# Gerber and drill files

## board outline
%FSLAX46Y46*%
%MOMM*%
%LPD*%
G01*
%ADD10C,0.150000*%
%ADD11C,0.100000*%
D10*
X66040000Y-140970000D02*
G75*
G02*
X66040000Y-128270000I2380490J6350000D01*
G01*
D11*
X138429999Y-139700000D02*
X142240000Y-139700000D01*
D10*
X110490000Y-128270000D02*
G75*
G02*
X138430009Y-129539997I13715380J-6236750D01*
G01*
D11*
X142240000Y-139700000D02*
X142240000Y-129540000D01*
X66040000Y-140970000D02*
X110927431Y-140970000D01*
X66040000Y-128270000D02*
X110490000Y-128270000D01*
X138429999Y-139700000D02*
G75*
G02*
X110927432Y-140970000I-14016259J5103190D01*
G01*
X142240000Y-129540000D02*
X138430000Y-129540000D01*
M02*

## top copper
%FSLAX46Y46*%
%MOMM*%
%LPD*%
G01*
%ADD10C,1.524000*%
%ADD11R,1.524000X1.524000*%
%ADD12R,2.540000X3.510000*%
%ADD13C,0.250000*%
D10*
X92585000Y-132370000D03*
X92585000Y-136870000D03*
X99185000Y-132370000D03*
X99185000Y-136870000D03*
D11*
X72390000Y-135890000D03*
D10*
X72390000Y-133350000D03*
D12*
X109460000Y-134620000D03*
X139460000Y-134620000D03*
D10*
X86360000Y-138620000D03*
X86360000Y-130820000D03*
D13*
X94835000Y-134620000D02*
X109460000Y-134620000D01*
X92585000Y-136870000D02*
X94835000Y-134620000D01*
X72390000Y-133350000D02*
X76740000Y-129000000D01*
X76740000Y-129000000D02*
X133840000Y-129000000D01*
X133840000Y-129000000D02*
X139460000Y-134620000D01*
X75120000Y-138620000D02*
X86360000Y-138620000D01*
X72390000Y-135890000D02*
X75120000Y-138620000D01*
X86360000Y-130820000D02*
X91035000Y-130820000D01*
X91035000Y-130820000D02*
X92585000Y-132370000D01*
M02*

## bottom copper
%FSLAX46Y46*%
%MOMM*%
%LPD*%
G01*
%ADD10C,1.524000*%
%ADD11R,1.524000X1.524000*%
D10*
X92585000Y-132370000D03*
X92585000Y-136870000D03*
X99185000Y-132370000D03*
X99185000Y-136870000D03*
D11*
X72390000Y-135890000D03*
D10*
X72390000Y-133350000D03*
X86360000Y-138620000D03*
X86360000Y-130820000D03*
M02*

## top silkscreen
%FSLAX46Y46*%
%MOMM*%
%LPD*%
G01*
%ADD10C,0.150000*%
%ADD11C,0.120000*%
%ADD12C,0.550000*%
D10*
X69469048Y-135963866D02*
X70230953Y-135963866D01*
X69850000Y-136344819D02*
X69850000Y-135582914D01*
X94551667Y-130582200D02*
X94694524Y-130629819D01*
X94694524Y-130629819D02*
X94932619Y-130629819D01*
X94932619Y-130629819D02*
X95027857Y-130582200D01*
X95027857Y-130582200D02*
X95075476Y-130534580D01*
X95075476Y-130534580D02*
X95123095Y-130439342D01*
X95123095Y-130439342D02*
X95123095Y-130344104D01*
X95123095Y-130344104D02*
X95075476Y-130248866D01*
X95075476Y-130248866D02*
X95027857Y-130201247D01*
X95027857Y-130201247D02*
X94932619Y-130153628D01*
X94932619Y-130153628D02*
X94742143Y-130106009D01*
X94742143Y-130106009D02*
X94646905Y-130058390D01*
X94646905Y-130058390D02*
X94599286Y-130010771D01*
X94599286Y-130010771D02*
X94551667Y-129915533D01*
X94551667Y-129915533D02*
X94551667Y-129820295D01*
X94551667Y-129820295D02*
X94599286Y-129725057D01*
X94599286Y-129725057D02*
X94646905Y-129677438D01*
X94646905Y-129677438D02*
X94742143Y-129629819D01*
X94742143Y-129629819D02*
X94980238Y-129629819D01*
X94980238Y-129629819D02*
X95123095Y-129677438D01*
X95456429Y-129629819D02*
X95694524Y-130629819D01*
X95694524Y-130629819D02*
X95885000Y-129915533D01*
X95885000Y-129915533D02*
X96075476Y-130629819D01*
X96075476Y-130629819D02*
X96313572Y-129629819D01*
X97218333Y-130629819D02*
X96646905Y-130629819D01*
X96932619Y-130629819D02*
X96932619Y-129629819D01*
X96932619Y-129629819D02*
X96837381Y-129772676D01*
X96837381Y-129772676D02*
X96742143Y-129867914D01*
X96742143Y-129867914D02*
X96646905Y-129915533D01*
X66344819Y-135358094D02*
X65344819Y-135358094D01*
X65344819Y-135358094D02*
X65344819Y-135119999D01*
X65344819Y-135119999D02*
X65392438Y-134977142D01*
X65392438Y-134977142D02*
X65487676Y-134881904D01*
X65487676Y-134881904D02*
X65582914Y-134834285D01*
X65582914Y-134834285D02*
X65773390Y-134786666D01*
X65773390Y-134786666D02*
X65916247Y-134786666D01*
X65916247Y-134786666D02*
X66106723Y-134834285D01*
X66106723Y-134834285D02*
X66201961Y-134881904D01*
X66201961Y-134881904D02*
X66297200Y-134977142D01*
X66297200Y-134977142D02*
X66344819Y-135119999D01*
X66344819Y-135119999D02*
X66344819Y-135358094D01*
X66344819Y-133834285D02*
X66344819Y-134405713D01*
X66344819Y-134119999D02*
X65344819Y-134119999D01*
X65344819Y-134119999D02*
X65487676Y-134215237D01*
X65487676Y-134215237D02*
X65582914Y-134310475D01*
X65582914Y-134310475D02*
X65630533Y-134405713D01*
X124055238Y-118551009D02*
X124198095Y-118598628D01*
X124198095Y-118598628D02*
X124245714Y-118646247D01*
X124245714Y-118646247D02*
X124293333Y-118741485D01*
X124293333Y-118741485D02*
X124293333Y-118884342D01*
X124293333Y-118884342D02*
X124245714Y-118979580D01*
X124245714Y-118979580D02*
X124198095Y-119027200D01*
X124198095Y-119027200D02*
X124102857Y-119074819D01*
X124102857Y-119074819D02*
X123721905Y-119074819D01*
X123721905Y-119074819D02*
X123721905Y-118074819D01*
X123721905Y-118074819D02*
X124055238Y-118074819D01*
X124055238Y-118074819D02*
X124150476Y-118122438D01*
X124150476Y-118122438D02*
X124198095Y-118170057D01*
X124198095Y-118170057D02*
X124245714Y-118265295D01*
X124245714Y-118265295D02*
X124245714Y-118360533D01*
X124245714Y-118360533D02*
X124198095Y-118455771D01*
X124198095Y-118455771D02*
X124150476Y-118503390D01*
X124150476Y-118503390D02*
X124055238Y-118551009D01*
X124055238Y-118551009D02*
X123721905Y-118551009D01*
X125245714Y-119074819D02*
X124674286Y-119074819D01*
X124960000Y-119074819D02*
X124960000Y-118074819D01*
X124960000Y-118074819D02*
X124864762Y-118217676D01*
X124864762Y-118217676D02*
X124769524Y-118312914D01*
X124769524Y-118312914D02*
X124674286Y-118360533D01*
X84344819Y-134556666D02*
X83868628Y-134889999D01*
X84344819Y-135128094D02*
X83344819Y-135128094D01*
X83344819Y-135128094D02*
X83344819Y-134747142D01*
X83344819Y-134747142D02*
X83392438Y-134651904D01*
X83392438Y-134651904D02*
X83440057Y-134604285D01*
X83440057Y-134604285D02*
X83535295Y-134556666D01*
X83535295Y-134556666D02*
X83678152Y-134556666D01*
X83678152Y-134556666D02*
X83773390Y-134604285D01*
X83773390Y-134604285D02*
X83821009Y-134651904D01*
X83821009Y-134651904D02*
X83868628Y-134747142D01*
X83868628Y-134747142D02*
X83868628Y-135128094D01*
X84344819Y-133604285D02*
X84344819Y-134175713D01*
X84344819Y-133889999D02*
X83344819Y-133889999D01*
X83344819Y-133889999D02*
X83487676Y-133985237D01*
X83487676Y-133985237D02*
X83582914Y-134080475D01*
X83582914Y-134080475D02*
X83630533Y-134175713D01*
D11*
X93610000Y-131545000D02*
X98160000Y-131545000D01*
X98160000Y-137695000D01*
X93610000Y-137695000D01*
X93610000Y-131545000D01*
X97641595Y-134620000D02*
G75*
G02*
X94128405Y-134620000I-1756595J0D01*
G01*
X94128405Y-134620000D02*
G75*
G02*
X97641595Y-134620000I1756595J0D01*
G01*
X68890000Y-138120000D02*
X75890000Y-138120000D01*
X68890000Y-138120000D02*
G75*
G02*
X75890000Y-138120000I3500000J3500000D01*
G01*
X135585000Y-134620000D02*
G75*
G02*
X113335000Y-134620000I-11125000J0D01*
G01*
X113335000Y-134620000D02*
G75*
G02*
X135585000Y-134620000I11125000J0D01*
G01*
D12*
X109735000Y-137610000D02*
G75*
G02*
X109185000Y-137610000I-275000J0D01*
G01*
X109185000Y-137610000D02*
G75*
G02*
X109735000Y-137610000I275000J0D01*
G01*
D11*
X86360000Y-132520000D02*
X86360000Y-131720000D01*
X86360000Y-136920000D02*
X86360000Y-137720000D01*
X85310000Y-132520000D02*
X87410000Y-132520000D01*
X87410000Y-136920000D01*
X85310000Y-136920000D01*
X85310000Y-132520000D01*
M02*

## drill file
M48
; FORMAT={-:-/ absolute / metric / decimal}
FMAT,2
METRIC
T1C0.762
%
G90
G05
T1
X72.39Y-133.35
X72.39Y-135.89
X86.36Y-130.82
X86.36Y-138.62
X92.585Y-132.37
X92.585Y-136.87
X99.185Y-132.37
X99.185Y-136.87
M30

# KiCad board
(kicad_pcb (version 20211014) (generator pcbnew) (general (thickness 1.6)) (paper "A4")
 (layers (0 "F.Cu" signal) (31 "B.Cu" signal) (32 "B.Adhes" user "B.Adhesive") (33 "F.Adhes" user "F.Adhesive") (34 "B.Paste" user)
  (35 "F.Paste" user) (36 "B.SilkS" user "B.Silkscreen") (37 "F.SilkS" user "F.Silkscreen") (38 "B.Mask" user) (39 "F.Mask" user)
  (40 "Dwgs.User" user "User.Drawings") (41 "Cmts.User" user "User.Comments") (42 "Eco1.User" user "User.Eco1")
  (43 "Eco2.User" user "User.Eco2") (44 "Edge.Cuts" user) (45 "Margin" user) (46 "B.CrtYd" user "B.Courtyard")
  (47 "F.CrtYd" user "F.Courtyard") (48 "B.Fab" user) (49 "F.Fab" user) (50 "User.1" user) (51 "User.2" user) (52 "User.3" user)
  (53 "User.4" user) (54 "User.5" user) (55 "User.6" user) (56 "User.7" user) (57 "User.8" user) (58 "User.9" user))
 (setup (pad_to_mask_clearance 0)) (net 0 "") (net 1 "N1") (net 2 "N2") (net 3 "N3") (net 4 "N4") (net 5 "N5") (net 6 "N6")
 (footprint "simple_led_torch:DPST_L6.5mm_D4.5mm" (layer "F.Cu") (at 95.885 134.62)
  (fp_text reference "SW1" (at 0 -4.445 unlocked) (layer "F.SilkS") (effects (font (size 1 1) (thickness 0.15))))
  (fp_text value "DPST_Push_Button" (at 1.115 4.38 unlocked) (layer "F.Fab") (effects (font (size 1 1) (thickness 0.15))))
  (fp_rect (start -2.275 -3.075) (end 2.275 3.075) (layer "F.SilkS") (width 0.12) (fill none))
  (fp_circle (center 0 0) (end 0.725 1.6) (layer "F.SilkS") (width 0.12) (fill none))
  (pad "1" thru_hole circle (at -3.3 -2.25) (size 1.524 1.524) (drill 0.762) (layers *.Cu *.Mask) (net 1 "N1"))
  (pad "2" thru_hole circle (at -3.3 2.25) (size 1.524 1.524) (drill 0.762) (layers *.Cu *.Mask) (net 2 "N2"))
  (pad "3" thru_hole circle (at 3.3 -2.25) (size 1.524 1.524) (drill 0.762) (layers *.Cu *.Mask) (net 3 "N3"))
  (pad "4" thru_hole circle (at 3.3 2.25) (size 1.524 1.524) (drill 0.762) (layers *.Cu *.Mask) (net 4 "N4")))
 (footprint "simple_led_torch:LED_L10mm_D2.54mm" (layer "F.Cu") (at 72.39 134.62 90)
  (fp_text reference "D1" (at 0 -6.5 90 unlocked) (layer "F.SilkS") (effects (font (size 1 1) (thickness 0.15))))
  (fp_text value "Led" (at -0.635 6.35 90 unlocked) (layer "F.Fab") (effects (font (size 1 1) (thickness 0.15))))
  (fp_line (start -3.5 -3.5) (end -3.5 3.5) (layer "F.SilkS") (width 0.12))
  (fp_arc (start -3.5 -3.5) (mid 4.949747 0) (end -3.5 3.5) (layer "F.SilkS") (width 0.12))
  (pad "1" thru_hole rect (at -1.27 0 90) (size 1.524 1.524) (drill 0.762) (layers *.Cu *.Mask) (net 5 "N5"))
  (pad "2" thru_hole circle (at 1.27 0 90) (size 1.524 1.524) (drill 0.762) (layers *.Cu *.Mask) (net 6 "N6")))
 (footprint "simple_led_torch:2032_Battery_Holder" (layer "F.Cu") (at 124.46 134.62)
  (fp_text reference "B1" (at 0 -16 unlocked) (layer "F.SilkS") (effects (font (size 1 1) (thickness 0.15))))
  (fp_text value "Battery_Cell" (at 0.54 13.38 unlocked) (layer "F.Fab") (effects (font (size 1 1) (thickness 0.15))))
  (fp_circle (center 0 0) (end 11.125 0) (layer "F.SilkS") (width 0.12) (fill none))
  (fp_circle (center -15 2.99) (end -14.5 2.99) (layer "F.SilkS") (width 0.1) (fill solid))
  (pad "1" smd rect (at -15 0) (size 2.54 3.51) (layers "F.Cu" "F.Paste" "F.Mask") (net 2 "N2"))
  (pad "2" smd rect (at 15 0) (size 2.54 3.51) (layers "F.Cu" "F.Paste" "F.Mask") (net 6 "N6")))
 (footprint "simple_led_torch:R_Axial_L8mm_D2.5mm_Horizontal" (layer "F.Cu") (at 86.36 138.62 90)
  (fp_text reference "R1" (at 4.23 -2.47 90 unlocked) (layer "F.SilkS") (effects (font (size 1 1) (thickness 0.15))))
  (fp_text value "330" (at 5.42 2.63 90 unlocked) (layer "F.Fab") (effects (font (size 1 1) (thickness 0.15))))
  (fp_line (start 6.1 0) (end 6.9 0) (layer "F.SilkS") (width 0.12))
  (fp_line (start 1.7 0) (end 0.9 0) (layer "F.SilkS") (width 0.12))
  (fp_rect (start 1.7 -1.05) (end 6.1 1.05) (layer "F.SilkS") (width 0.12) (fill none))
  (pad "1" thru_hole circle (at 0 0 90) (size 1.524 1.524) (drill 0.762) (layers *.Cu *.Mask) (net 5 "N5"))
  (pad "2" thru_hole circle (at 7.8 0 90) (size 1.524 1.524) (drill 0.762) (layers *.Cu *.Mask) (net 1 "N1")))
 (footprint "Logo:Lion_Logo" (layer "B.Cu") (at 125 132 180)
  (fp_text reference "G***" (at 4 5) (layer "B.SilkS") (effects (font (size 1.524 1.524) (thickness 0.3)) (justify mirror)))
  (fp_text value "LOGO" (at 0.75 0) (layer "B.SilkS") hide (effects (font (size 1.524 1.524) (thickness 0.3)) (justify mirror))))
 (gr_arc (start 66.04 140.97) (mid 61.638952 134.62) (end 66.04 128.27) (layer "Edge.Cuts") (width 0.15))
 (gr_line (start 138.429999 139.7) (end 142.24 139.7) (layer "Edge.Cuts") (width 0.1))
 (gr_arc (start 110.49 128.27) (mid 124.889523 119.455486) (end 138.43 129.54) (layer "Edge.Cuts") (width 0.15))
 (gr_line (start 142.24 139.7) (end 142.24 129.54) (layer "Edge.Cuts") (width 0.1))
 (gr_line (start 66.04 140.97) (end 110.927431 140.97) (layer "Edge.Cuts") (width 0.1))
 (gr_line (start 66.04 128.27) (end 110.49 128.27) (layer "Edge.Cuts") (width 0.1))
 (gr_arc (start 138.429999 139.7) (mid 125.101807 149.4973) (end 110.927431 140.97) (layer "Edge.Cuts") (width 0.1))
 (gr_line (start 142.24 129.54) (end 138.43 129.54) (layer "Edge.Cuts") (width 0.1))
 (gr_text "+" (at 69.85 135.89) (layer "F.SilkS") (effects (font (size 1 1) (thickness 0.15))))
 (segment (start 94.835 134.62) (end 109.46 134.62) (width 0.25) (layer "F.Cu") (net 2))
 (segment (start 92.585 136.87) (end 94.835 134.62) (width 0.25) (layer "F.Cu") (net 2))
 (segment (start 72.39 133.35) (end 76.74 129) (width 0.25) (layer "F.Cu") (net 6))
 (segment (start 76.74 129) (end 133.84 129) (width 0.25) (layer "F.Cu") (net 6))
 (segment (start 133.84 129) (end 139.46 134.62) (width 0.25) (layer "F.Cu") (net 6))
 (segment (start 75.12 138.62) (end 86.36 138.62) (width 0.25) (layer "F.Cu") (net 5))
 (segment (start 72.39 135.89) (end 75.12 138.62) (width 0.25) (layer "F.Cu") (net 5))
 (segment (start 86.36 130.82) (end 91.035 130.82) (width 0.25) (layer "F.Cu") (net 1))
 (segment (start 91.035 130.82) (end 92.585 132.37) (width 0.25) (layer "F.Cu") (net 1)))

